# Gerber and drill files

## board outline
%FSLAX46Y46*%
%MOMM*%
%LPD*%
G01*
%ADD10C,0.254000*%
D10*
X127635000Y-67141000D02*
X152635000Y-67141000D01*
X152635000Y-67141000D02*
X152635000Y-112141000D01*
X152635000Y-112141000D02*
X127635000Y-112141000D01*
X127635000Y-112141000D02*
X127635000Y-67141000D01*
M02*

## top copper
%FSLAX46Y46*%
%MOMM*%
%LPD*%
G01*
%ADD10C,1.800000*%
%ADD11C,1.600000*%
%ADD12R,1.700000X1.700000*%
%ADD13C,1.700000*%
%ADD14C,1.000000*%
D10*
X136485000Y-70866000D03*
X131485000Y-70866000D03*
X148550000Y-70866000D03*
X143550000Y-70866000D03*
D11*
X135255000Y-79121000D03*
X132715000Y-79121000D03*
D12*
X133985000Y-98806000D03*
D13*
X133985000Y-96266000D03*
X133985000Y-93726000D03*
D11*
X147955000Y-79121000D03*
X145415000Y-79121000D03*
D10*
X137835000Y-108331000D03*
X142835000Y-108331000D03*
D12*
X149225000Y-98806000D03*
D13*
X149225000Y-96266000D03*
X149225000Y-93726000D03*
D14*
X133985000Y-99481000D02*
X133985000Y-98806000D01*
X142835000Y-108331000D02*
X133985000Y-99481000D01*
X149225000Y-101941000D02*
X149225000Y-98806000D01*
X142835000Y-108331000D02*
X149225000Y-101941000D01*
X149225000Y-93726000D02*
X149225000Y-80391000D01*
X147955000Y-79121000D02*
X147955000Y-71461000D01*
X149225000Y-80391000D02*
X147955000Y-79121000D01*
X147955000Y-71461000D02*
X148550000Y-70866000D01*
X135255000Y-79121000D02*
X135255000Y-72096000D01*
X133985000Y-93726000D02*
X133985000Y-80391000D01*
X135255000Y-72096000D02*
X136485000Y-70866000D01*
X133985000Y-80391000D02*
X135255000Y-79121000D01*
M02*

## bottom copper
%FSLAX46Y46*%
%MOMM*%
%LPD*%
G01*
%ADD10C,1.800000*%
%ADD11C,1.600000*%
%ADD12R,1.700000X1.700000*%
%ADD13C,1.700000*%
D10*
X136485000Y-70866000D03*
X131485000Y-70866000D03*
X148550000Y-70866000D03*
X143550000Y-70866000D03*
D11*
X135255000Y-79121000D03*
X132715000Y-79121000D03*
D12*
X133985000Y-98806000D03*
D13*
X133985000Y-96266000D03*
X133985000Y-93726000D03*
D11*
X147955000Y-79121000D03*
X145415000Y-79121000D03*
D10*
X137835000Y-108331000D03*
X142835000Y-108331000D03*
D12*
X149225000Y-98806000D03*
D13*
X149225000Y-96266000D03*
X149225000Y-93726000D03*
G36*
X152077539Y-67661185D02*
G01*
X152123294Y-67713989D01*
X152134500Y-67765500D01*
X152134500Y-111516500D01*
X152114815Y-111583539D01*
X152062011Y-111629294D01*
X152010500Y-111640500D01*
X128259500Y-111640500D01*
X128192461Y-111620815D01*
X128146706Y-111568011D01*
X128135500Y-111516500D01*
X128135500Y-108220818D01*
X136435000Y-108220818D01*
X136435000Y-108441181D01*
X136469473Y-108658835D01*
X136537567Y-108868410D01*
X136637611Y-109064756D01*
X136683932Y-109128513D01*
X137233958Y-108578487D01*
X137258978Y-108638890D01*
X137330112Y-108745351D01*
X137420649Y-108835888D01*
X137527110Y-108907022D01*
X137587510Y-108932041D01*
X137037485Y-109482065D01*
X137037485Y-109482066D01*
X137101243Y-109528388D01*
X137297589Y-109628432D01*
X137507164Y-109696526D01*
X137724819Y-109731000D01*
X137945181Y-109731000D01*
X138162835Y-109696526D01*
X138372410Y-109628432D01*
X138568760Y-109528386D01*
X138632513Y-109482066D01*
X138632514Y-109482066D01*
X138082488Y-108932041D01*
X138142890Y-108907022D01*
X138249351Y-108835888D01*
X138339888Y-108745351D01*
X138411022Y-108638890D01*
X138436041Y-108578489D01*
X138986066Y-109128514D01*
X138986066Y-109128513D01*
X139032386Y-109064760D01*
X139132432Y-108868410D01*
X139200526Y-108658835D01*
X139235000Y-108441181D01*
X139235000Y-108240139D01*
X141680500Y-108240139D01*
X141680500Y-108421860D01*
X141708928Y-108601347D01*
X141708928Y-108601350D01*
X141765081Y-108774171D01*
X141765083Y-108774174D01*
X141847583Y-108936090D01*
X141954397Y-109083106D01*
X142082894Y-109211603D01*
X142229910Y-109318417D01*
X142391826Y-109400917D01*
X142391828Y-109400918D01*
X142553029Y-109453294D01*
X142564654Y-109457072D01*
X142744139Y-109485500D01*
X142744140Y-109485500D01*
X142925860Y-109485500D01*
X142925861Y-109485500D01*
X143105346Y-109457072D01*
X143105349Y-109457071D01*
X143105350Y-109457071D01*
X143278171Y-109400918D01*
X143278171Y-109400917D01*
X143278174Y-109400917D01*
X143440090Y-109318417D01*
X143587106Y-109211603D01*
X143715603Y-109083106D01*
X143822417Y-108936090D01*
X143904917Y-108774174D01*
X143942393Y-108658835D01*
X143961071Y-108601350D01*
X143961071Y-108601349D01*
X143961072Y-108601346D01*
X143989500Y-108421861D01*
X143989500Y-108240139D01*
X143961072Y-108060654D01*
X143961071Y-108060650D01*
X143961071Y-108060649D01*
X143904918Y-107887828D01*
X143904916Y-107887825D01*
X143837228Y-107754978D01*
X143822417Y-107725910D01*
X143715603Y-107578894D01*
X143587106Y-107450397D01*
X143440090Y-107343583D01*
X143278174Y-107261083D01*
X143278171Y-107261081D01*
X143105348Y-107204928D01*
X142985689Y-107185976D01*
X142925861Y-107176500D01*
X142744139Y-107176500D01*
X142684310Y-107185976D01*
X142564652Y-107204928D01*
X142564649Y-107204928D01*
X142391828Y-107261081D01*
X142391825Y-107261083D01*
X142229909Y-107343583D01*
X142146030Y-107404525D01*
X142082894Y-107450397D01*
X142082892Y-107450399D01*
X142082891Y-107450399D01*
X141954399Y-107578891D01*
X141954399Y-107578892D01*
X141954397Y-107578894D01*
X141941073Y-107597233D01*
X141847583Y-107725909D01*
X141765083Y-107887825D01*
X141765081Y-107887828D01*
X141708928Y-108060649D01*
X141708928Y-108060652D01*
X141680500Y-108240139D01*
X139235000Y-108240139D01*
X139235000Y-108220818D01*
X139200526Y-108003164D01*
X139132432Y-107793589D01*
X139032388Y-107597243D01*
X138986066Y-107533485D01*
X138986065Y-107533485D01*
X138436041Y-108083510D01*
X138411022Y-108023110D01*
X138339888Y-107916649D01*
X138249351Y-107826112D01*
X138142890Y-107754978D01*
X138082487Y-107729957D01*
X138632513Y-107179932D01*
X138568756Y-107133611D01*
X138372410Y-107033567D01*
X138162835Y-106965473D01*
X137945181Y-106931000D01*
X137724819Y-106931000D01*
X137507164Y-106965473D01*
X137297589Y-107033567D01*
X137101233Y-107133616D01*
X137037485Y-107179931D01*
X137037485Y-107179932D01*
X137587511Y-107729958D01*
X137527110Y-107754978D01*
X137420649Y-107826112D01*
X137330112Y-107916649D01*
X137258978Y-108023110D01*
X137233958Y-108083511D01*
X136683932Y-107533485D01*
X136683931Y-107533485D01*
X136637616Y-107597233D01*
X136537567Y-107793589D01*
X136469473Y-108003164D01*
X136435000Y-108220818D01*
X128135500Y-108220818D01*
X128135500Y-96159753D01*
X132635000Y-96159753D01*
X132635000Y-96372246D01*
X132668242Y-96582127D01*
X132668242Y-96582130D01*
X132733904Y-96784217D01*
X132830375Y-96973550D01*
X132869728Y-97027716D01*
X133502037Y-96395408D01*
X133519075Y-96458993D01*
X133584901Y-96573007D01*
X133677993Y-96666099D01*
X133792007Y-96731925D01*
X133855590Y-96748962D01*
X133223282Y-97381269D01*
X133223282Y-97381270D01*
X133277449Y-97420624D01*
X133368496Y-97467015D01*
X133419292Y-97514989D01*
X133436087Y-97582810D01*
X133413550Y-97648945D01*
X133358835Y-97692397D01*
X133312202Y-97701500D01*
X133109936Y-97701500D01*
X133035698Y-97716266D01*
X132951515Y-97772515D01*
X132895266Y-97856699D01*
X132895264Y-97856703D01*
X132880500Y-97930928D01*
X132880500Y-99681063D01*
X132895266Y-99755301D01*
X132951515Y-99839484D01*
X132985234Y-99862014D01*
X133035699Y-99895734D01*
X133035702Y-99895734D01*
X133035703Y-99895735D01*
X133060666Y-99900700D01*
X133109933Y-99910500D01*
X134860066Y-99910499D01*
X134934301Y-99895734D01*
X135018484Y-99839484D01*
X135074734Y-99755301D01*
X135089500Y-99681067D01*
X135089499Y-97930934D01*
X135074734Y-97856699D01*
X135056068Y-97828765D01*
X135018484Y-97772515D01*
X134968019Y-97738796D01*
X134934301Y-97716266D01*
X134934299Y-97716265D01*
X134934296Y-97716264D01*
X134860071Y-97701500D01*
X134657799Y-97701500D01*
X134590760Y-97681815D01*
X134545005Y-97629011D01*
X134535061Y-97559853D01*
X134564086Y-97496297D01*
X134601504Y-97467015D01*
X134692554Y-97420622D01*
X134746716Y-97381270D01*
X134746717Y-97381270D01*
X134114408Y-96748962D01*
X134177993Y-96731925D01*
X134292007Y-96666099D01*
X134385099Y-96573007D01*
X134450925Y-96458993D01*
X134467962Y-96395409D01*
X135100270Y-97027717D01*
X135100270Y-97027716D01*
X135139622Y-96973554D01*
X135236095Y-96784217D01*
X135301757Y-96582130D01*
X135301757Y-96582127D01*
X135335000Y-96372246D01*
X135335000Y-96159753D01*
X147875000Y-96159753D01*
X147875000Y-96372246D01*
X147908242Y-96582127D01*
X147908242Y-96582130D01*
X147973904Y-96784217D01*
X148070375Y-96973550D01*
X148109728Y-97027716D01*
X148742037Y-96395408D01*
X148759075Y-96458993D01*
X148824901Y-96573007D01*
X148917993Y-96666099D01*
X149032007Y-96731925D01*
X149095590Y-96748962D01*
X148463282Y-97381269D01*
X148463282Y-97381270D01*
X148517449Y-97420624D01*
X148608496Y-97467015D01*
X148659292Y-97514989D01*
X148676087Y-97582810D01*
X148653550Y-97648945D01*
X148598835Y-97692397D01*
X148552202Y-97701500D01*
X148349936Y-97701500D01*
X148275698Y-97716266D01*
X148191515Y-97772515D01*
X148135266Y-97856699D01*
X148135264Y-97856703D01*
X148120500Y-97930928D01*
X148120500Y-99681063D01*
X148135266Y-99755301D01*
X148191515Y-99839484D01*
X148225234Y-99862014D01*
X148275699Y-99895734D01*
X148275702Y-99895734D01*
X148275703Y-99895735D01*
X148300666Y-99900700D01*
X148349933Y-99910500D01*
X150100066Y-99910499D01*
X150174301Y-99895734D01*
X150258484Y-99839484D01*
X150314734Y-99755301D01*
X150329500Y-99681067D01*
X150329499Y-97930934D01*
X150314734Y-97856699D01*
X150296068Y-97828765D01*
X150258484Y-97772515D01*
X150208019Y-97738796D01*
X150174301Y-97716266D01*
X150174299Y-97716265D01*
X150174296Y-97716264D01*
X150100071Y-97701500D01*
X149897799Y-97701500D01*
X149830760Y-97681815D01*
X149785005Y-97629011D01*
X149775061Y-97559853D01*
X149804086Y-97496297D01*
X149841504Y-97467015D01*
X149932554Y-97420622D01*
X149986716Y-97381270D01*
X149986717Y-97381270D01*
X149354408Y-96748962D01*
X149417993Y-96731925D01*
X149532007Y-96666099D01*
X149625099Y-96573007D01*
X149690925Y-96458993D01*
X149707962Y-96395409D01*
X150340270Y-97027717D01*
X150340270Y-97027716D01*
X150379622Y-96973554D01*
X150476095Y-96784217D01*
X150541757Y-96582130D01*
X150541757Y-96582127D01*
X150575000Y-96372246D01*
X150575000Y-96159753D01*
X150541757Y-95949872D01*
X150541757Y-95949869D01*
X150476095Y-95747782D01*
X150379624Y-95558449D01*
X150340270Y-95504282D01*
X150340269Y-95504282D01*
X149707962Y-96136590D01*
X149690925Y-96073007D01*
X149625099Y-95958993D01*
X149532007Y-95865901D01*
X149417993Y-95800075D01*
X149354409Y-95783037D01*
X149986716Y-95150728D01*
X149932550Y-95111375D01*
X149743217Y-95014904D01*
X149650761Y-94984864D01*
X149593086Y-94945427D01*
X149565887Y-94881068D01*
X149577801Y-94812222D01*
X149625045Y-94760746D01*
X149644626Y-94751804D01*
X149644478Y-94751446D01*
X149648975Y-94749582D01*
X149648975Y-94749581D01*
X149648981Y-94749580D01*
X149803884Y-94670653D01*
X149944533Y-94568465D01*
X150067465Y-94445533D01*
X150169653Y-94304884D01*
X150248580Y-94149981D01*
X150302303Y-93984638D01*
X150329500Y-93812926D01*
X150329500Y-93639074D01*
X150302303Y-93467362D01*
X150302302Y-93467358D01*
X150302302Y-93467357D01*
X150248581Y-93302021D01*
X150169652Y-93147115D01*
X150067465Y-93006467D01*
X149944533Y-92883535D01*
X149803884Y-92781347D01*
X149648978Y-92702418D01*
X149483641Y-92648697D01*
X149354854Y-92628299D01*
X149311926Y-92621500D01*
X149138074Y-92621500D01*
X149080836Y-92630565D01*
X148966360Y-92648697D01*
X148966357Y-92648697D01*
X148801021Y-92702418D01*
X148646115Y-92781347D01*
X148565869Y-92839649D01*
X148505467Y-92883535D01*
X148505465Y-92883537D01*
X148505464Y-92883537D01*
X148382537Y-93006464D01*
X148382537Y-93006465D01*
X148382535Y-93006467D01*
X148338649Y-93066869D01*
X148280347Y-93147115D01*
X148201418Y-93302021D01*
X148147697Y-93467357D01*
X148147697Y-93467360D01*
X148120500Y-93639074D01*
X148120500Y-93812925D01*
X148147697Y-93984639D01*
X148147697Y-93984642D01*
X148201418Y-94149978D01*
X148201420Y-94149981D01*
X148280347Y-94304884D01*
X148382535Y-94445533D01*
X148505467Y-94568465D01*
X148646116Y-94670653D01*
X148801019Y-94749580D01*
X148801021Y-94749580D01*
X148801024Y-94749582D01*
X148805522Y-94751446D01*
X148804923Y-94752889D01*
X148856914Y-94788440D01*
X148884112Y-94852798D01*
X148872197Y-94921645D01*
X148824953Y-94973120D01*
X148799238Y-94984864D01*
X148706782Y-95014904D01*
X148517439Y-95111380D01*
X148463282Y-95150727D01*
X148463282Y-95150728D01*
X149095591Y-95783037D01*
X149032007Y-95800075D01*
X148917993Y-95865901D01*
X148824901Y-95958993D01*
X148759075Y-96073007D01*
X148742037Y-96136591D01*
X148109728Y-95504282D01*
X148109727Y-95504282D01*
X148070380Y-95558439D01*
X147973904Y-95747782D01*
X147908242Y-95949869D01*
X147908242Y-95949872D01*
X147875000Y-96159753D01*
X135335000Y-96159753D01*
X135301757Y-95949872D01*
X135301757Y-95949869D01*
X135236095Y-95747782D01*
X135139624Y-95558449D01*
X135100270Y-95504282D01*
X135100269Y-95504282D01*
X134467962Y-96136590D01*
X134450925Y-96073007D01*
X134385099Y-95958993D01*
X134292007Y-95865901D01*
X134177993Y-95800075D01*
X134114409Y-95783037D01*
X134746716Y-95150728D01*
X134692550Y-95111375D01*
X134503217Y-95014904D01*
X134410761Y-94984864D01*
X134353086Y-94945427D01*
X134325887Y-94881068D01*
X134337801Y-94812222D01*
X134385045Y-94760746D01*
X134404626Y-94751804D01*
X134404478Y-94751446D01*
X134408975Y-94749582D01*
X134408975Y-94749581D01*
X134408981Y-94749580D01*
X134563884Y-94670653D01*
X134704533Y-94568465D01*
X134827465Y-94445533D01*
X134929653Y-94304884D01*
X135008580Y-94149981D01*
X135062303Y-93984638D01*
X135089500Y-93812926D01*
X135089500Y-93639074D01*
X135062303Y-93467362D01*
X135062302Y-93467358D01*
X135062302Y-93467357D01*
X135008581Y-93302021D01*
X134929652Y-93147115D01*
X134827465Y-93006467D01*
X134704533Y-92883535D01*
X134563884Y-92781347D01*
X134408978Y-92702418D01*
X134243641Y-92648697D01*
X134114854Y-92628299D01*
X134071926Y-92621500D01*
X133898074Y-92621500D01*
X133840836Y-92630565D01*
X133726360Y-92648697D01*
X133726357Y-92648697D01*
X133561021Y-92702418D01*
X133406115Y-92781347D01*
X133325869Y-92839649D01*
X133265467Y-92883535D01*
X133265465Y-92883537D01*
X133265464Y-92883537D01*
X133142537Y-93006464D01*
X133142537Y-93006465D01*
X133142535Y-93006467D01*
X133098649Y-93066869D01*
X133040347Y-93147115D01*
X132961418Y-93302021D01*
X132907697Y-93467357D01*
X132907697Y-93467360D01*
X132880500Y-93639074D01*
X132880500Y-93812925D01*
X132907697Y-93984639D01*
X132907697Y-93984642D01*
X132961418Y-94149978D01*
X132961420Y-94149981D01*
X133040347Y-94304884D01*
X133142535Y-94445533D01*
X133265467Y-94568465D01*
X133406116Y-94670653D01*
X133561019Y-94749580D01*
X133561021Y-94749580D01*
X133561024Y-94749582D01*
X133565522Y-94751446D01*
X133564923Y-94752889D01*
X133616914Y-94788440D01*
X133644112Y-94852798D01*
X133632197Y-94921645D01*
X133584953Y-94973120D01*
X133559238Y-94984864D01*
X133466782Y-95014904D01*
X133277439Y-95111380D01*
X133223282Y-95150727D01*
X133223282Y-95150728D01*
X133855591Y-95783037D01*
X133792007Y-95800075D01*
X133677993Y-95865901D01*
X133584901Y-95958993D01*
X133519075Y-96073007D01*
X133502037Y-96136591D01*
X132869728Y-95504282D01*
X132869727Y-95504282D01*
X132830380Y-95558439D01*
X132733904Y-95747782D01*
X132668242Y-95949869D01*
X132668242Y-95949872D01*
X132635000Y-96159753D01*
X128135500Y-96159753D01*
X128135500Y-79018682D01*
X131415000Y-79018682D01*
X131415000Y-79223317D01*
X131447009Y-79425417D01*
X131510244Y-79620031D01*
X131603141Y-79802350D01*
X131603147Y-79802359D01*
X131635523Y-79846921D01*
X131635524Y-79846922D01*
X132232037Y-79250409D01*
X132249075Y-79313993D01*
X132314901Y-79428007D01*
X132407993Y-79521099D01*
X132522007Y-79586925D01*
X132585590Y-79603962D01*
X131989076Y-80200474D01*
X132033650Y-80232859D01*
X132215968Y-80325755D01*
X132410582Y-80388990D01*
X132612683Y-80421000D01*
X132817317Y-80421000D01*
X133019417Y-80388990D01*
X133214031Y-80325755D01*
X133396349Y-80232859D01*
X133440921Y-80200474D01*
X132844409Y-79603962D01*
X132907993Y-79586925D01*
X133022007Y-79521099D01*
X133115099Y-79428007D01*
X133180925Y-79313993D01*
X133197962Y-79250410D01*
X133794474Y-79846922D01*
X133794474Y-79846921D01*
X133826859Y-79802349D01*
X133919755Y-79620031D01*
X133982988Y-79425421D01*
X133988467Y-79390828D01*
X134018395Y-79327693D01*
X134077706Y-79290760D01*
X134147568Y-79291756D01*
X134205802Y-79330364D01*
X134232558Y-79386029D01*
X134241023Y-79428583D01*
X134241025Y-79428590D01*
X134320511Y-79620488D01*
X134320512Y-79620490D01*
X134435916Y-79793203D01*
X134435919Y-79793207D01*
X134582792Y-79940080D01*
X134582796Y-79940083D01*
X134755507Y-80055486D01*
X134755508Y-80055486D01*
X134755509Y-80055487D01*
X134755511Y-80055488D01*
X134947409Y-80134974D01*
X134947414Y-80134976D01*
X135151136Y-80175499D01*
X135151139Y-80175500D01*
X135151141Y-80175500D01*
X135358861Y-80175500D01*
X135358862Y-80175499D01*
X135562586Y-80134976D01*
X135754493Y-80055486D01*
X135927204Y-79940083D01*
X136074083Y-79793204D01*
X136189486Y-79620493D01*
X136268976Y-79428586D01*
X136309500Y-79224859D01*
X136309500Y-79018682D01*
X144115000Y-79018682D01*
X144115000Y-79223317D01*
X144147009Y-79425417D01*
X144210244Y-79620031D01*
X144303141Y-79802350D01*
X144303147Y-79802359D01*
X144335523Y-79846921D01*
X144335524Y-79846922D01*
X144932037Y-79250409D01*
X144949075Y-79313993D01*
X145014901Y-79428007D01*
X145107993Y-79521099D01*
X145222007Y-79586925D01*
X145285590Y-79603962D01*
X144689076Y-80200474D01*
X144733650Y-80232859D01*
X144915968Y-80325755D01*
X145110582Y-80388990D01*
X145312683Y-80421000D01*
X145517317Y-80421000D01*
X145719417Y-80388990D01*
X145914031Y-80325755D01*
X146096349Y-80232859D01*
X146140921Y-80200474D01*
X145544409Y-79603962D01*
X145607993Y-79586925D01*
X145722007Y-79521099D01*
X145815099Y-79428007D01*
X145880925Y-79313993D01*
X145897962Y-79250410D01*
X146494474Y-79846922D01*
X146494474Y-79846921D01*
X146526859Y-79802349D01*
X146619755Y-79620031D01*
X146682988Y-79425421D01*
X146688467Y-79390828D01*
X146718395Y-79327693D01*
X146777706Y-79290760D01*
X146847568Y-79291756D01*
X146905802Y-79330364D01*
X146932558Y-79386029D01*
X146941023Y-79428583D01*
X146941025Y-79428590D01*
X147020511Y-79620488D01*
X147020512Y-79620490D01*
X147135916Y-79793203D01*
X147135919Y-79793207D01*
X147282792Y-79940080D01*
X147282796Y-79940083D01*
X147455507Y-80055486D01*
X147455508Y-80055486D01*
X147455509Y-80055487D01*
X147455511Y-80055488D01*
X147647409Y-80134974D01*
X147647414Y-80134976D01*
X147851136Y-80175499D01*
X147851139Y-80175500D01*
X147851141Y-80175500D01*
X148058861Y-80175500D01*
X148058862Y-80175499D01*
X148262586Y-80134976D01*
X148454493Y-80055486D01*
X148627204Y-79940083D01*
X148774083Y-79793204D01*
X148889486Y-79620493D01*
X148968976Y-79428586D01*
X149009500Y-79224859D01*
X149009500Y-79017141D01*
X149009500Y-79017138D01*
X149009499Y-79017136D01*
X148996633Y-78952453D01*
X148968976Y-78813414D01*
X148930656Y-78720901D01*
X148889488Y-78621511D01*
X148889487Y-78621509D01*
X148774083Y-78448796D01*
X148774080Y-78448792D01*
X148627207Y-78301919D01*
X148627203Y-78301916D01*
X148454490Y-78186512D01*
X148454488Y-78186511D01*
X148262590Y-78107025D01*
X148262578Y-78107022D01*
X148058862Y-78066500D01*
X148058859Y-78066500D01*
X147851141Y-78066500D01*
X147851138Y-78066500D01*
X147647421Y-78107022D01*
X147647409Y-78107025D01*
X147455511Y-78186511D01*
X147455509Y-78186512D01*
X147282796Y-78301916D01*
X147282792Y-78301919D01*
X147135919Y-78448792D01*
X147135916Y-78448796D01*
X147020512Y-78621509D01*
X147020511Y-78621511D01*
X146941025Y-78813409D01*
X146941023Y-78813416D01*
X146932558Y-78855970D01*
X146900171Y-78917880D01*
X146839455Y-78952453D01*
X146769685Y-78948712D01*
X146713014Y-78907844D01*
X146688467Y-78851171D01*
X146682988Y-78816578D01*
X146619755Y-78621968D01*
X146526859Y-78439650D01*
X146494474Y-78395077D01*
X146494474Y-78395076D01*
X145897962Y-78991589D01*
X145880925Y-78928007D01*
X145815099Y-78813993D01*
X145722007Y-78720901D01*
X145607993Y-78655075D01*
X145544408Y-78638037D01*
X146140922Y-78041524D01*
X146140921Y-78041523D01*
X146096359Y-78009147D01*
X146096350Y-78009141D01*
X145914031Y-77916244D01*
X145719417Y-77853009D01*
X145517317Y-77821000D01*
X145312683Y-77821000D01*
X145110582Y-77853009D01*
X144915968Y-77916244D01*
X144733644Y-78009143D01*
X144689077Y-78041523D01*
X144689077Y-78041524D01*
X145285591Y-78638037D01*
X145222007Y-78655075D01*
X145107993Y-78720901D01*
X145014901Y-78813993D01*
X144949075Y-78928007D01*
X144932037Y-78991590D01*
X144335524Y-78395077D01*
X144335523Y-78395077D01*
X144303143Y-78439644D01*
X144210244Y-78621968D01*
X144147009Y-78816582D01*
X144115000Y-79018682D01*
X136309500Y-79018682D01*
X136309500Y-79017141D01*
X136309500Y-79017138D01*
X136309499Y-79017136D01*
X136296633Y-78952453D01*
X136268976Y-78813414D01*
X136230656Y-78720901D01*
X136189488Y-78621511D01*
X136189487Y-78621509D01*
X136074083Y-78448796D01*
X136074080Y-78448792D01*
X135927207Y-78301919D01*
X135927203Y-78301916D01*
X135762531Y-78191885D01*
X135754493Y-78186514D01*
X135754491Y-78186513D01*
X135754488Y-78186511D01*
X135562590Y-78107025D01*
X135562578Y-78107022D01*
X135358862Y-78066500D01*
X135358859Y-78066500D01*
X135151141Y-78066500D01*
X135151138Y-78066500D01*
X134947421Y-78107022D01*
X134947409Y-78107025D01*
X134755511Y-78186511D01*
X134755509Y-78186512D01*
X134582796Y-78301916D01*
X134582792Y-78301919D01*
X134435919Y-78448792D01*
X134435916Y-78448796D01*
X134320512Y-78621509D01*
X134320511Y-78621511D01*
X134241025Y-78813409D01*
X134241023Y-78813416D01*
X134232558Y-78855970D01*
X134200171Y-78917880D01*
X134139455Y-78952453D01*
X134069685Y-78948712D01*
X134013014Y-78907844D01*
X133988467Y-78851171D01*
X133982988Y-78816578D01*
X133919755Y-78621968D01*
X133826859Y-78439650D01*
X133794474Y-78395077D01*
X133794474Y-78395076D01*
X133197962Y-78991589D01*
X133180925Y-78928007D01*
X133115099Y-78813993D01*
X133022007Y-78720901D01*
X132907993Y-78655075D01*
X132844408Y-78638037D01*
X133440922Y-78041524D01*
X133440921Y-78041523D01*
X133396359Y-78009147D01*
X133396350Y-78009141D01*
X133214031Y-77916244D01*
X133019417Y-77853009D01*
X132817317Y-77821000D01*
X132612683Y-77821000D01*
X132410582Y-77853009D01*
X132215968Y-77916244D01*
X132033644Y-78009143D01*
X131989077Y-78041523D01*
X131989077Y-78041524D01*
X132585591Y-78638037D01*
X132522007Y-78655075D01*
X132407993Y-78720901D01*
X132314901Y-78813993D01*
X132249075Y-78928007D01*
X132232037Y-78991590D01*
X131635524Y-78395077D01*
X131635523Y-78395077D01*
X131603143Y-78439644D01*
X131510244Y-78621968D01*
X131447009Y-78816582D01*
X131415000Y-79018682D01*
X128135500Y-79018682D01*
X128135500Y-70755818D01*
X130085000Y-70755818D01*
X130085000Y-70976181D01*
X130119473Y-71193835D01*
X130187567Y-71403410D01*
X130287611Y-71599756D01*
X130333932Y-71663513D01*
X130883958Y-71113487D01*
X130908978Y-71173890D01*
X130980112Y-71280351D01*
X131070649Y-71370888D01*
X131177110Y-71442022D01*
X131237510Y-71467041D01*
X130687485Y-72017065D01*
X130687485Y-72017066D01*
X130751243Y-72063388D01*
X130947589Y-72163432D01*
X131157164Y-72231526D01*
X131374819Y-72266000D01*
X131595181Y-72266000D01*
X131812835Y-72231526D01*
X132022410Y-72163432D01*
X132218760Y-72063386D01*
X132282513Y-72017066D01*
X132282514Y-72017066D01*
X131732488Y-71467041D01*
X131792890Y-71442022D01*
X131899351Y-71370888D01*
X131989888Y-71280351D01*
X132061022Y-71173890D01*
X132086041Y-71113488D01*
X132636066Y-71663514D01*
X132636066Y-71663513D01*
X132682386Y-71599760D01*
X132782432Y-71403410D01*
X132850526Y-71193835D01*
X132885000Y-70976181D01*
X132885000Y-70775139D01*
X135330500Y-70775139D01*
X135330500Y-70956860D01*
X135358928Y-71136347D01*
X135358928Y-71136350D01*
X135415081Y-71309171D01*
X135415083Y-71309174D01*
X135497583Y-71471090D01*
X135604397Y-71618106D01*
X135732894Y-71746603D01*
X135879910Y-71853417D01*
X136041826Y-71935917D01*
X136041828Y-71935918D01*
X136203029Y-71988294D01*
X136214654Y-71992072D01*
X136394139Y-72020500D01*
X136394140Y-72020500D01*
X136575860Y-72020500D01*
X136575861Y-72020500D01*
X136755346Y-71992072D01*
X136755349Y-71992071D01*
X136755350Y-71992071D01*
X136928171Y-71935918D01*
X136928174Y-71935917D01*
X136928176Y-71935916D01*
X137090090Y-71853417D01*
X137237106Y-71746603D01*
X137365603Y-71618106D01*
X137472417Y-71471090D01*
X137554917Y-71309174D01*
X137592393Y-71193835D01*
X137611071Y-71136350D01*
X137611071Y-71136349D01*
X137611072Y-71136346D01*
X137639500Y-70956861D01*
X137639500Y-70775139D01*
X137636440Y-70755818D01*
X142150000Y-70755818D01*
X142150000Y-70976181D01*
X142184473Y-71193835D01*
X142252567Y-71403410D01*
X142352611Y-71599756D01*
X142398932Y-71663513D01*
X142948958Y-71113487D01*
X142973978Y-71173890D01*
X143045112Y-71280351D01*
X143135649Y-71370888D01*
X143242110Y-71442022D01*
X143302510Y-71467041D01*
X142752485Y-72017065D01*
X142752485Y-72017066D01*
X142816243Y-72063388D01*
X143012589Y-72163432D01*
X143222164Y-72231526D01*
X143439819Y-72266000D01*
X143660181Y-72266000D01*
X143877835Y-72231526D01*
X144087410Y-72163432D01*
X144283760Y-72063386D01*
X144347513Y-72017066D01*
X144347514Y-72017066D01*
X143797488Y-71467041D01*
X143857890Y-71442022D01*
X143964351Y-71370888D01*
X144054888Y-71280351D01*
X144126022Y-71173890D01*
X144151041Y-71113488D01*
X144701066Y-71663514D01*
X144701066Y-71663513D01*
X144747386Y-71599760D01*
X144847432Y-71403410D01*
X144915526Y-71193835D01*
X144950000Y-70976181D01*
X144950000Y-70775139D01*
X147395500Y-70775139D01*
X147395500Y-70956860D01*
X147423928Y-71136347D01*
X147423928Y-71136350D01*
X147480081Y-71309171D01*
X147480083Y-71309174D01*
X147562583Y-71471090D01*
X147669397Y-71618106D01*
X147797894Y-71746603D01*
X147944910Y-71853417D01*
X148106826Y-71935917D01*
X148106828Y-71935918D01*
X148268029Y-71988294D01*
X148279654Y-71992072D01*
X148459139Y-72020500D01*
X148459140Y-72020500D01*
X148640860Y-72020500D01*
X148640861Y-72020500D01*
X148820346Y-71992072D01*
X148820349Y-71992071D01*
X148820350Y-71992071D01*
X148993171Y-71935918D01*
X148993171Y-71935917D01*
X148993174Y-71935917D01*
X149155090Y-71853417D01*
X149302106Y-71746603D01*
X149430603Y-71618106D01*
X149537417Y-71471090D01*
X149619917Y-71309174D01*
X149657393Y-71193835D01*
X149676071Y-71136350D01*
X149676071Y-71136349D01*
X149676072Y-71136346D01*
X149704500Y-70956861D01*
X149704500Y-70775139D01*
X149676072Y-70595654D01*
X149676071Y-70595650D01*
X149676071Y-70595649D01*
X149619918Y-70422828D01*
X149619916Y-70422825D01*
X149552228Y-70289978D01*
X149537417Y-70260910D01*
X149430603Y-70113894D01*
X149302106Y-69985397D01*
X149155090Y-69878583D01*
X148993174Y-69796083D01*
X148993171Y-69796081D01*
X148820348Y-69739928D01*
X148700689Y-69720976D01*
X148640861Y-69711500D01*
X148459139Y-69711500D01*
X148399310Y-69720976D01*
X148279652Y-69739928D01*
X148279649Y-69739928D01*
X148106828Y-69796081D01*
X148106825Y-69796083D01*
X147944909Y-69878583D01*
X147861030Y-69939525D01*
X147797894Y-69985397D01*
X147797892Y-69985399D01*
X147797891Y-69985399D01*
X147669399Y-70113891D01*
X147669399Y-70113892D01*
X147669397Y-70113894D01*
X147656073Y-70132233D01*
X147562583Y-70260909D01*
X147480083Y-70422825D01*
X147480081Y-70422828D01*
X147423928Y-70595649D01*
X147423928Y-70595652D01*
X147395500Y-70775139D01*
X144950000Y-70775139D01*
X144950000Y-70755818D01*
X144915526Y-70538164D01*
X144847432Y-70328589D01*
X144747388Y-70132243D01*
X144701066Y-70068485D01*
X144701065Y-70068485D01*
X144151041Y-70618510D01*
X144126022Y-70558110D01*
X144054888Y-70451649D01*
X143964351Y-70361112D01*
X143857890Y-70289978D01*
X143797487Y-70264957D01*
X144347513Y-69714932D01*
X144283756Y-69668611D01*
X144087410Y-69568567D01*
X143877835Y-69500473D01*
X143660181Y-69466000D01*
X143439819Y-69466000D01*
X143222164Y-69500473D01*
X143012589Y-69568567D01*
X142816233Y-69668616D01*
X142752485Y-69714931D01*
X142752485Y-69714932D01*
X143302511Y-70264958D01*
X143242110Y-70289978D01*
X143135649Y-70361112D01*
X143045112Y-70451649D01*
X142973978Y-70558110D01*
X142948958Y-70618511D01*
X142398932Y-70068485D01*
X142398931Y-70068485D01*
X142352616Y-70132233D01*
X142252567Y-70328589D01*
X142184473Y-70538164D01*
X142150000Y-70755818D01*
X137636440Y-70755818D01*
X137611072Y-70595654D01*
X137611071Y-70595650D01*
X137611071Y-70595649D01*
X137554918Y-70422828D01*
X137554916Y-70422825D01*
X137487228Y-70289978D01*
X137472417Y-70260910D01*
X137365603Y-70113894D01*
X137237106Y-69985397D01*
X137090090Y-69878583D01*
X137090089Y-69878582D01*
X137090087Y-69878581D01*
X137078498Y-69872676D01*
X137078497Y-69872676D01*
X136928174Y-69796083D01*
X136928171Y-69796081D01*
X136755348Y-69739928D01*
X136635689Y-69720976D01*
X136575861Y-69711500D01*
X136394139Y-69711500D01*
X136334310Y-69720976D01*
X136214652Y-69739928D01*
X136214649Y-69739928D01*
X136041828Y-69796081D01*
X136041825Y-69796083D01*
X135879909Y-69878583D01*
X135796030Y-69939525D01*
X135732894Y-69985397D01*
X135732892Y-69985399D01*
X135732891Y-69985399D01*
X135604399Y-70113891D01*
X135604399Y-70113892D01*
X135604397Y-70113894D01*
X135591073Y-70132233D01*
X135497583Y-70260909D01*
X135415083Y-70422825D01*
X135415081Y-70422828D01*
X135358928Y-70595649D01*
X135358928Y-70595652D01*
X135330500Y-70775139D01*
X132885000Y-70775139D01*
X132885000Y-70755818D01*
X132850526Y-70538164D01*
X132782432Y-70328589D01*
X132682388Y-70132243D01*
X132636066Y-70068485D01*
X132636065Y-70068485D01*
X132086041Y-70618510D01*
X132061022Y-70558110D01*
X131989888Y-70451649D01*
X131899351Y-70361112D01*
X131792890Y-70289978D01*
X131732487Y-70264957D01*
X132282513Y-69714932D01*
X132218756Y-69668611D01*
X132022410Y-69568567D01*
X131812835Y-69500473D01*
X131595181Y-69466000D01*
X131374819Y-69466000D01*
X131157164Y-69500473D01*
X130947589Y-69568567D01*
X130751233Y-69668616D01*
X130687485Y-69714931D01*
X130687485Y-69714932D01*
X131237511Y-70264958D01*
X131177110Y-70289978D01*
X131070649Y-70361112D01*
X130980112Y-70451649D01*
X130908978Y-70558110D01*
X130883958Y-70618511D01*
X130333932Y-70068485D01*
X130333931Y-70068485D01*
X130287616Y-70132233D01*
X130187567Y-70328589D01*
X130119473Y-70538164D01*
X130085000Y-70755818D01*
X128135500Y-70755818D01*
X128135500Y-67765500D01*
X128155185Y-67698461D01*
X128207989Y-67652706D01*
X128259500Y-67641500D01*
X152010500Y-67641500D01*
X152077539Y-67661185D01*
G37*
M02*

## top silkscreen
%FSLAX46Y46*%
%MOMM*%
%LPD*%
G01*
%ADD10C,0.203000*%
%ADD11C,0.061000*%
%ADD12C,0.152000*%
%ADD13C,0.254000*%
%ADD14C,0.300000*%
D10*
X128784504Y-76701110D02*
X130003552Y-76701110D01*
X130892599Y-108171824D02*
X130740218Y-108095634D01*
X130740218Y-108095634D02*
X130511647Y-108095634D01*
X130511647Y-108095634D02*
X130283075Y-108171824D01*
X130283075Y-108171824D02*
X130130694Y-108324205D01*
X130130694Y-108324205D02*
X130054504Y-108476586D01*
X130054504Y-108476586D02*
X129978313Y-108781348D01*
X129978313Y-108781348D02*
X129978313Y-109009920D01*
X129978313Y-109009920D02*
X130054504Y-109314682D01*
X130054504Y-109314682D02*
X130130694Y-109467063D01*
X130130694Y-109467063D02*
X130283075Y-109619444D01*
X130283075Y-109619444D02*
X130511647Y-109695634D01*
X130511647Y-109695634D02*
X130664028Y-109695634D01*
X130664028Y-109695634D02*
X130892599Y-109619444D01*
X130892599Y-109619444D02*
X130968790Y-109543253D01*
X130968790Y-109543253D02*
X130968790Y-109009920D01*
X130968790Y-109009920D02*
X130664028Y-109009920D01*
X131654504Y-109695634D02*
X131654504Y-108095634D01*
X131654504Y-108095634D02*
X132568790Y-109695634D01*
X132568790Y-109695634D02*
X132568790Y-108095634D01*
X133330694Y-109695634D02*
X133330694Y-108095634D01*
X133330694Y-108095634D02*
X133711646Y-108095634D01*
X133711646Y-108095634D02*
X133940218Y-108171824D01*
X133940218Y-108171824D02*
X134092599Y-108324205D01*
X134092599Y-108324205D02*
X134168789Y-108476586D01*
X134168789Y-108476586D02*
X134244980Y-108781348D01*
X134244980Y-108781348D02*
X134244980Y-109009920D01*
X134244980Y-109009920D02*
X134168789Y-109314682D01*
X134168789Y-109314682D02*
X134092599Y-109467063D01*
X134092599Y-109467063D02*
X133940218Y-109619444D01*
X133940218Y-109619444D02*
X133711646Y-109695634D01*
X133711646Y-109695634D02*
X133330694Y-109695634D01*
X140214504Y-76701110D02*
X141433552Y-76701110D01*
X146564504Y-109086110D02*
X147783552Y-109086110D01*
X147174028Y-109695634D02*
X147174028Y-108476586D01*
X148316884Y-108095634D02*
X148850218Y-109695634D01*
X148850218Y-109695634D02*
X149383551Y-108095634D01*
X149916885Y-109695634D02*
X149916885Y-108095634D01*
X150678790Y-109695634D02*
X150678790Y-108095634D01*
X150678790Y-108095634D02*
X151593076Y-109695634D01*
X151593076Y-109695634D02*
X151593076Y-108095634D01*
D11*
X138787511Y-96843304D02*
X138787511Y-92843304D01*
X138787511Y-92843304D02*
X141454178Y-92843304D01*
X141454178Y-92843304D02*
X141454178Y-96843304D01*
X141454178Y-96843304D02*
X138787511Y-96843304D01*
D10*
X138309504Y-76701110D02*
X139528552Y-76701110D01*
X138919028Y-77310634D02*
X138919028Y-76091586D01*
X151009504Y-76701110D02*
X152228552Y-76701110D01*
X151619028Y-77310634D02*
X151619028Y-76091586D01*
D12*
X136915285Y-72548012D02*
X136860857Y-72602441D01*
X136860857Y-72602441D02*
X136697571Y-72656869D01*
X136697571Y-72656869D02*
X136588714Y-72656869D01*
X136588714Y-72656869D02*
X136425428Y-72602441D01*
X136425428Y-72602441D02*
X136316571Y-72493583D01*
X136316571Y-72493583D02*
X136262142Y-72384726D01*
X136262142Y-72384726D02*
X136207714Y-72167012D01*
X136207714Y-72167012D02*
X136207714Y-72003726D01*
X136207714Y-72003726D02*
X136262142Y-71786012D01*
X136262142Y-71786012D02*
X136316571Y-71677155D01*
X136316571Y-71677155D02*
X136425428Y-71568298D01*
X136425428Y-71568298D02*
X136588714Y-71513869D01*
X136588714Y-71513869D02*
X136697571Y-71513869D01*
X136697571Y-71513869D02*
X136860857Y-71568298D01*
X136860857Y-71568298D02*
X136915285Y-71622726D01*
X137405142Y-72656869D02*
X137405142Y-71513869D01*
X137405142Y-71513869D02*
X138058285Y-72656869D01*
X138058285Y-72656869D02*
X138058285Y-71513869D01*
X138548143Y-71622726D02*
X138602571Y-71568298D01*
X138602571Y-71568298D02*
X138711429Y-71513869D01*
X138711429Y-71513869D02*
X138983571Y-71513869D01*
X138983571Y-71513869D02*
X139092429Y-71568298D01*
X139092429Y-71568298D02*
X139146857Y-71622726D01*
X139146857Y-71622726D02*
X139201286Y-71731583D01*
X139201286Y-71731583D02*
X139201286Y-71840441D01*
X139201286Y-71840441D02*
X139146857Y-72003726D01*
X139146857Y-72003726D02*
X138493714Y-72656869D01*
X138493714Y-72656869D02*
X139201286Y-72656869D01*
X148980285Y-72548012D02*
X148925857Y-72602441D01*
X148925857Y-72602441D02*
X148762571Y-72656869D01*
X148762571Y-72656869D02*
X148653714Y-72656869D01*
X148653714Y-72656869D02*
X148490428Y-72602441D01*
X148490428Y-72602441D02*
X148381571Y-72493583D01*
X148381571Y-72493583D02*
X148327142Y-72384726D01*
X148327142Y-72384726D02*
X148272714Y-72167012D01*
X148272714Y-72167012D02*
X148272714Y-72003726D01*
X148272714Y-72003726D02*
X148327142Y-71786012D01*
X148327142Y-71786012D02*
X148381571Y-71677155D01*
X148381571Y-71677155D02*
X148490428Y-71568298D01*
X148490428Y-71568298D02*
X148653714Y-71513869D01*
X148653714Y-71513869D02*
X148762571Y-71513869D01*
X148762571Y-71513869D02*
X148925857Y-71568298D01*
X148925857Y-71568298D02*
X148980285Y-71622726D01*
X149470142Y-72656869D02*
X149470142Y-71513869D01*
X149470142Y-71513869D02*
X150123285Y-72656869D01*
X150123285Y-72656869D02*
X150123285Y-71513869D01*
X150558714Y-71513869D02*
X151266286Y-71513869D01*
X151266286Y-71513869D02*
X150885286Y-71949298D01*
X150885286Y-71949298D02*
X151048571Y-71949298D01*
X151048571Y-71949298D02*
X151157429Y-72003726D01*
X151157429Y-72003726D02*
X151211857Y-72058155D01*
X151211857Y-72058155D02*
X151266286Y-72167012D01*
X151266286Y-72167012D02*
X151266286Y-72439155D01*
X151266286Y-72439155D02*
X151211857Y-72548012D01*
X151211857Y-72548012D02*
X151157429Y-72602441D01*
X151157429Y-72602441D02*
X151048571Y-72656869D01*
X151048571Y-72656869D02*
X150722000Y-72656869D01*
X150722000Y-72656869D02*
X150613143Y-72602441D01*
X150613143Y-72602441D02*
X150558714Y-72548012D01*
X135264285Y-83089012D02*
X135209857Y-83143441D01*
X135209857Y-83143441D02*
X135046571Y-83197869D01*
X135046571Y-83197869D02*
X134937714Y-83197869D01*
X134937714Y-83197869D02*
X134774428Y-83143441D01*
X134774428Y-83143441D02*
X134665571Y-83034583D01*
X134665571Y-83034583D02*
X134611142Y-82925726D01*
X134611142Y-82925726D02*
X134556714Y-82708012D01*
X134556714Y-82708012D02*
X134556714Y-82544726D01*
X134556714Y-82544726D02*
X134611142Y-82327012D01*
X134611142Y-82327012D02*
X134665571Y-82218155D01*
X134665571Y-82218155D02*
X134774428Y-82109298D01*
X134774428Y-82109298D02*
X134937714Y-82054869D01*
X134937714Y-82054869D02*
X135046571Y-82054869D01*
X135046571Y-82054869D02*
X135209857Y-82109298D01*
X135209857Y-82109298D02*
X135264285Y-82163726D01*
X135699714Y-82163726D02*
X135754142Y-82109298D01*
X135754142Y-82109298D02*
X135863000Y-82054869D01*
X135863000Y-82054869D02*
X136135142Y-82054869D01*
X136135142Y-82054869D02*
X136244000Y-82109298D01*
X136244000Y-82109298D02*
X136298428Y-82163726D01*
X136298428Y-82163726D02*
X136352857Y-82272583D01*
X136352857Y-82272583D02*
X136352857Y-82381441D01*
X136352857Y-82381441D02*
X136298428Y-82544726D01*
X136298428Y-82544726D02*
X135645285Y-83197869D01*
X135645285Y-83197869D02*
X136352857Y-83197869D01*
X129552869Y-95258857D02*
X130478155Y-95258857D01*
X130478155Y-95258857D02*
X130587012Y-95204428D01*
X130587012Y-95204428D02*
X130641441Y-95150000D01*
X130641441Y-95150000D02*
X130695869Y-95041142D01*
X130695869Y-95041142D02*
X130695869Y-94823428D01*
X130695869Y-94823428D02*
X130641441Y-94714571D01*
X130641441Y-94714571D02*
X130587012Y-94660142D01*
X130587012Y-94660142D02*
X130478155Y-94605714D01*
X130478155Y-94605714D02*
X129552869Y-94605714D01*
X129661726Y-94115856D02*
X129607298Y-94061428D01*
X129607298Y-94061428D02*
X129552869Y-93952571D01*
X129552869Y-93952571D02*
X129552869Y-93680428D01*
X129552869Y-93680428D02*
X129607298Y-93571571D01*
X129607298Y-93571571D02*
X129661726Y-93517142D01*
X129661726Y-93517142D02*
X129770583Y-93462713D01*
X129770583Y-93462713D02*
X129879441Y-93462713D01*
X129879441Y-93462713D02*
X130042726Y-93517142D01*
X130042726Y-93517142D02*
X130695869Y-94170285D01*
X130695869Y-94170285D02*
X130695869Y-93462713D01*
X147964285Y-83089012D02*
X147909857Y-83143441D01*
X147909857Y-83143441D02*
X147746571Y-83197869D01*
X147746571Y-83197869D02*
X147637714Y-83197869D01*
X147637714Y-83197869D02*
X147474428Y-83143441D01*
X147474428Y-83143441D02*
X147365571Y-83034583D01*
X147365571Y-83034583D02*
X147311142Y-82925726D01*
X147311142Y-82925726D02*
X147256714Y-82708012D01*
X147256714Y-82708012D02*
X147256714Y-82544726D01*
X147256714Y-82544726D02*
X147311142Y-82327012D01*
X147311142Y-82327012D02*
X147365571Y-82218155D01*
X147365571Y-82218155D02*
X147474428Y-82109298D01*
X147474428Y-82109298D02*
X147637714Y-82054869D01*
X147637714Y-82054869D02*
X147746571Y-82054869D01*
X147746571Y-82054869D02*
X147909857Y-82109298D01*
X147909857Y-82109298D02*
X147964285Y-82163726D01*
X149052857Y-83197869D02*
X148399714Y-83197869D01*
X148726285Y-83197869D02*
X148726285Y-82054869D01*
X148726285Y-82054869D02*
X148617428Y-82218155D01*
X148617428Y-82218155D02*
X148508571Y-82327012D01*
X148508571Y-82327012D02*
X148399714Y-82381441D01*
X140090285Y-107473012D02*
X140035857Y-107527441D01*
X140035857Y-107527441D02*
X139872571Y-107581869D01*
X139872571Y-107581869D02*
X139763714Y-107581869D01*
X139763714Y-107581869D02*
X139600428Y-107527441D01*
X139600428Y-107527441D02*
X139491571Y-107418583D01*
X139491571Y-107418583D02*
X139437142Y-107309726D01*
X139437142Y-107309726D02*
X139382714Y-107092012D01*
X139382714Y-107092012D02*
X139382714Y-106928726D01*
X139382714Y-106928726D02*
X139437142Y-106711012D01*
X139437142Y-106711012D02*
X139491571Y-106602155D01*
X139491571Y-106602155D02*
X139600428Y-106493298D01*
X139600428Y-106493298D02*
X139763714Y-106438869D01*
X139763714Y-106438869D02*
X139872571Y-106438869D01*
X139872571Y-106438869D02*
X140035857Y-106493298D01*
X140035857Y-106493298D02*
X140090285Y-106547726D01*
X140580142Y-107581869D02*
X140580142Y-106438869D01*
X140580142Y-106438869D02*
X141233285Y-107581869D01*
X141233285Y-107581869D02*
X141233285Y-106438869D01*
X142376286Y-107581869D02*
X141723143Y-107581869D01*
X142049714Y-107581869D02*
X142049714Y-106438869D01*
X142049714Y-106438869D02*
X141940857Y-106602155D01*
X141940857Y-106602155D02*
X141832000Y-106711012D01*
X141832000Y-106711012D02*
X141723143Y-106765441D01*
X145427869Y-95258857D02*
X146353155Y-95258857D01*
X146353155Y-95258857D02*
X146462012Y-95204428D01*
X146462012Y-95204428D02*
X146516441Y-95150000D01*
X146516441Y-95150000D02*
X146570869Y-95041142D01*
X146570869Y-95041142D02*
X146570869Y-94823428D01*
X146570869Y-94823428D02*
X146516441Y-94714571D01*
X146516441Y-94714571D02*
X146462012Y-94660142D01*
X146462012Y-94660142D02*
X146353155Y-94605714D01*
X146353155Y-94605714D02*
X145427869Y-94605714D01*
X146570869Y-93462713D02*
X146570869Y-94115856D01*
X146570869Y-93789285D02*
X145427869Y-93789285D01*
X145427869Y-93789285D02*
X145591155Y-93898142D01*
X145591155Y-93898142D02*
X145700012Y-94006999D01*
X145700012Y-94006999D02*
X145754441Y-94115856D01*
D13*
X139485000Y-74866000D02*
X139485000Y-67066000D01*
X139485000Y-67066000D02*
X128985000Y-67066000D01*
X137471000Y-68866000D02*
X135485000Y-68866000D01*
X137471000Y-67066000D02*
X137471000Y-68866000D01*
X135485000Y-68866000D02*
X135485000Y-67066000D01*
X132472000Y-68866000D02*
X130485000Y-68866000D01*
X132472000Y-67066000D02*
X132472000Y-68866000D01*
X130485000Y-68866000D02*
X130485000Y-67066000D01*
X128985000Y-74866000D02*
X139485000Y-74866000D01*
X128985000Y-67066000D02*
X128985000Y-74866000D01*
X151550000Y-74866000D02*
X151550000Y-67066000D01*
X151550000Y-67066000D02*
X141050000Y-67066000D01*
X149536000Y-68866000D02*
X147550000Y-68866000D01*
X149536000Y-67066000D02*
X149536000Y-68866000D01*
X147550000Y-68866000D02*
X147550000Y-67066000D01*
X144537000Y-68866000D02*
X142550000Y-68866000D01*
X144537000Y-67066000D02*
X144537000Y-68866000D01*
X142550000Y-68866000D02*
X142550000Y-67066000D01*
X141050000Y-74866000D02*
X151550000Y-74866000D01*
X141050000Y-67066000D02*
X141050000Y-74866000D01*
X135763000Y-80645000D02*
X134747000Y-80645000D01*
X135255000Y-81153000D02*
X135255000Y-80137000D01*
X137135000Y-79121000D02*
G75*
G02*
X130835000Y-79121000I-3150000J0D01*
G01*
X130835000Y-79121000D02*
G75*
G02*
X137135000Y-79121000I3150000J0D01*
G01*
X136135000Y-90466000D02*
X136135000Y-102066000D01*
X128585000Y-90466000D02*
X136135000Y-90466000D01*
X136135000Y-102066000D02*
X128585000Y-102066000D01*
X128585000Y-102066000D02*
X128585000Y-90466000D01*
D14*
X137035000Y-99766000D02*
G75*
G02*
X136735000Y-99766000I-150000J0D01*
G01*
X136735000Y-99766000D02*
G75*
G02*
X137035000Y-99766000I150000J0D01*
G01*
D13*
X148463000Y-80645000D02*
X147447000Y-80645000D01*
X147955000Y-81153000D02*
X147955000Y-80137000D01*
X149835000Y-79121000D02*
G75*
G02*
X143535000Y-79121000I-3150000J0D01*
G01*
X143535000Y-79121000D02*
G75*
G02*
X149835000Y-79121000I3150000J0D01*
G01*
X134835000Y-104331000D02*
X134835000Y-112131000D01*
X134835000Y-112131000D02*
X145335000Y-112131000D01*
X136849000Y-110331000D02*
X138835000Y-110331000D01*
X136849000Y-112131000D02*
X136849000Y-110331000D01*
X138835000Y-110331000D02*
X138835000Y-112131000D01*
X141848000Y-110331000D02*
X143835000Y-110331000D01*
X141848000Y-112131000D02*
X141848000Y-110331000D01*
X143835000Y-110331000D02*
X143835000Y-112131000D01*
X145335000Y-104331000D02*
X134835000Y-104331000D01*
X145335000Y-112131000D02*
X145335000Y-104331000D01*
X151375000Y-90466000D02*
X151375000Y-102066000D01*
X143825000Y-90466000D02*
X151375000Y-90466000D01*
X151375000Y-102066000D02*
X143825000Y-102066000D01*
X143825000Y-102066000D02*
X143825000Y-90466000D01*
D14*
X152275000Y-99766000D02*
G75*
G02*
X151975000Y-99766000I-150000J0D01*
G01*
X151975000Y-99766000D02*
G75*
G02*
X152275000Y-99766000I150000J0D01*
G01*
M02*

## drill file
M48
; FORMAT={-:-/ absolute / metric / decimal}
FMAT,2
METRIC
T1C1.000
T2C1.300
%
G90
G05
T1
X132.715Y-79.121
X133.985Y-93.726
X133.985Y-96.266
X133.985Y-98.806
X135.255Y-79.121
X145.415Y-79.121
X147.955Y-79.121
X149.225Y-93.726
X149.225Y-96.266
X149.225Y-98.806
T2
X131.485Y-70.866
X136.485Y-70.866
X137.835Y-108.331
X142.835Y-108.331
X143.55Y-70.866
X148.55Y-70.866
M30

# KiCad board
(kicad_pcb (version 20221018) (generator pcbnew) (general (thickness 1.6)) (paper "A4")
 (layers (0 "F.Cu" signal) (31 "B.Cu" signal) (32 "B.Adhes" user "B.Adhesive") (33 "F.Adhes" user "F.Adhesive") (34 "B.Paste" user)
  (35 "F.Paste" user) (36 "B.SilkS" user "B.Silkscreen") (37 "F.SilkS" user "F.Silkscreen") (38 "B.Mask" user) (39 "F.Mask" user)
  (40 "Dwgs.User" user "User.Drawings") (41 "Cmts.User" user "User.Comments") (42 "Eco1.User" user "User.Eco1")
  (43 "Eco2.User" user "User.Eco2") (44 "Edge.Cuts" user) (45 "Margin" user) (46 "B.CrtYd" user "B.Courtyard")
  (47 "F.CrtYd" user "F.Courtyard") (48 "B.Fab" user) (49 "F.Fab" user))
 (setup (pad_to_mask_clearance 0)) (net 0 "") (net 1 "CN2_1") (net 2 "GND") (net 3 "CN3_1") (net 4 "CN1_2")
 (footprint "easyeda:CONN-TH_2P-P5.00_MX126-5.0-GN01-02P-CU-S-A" (layer "F.Cu") (at 133.985 70.866 180)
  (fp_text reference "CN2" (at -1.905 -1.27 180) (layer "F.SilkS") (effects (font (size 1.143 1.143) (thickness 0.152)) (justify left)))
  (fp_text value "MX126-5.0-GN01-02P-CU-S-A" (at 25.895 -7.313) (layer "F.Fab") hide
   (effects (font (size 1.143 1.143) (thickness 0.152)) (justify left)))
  (fp_line (start -5.5 -4) (end -5.5 3.8) (stroke (width 0.254) (type solid)) (layer "F.SilkS"))
  (fp_line (start -5.5 3.8) (end 5 3.8) (stroke (width 0.254) (type solid)) (layer "F.SilkS"))
  (fp_line (start -3.486 2) (end -1.5 2) (stroke (width 0.254) (type solid)) (layer "F.SilkS"))
  (fp_line (start -3.486 3.8) (end -3.486 2) (stroke (width 0.254) (type solid)) (layer "F.SilkS"))
  (fp_line (start -1.5 2) (end -1.5 3.8) (stroke (width 0.254) (type solid)) (layer "F.SilkS"))
  (fp_line (start 1.513 2) (end 3.5 2) (stroke (width 0.254) (type solid)) (layer "F.SilkS"))
  (fp_line (start 1.513 3.8) (end 1.513 2) (stroke (width 0.254) (type solid)) (layer "F.SilkS"))
  (fp_line (start 3.5 2) (end 3.5 3.8) (stroke (width 0.254) (type solid)) (layer "F.SilkS"))
  (fp_line (start 5 -4) (end -5.5 -4) (stroke (width 0.254) (type solid)) (layer "F.SilkS"))
  (fp_line (start 5 3.8) (end 5 -4) (stroke (width 0.254) (type solid)) (layer "F.SilkS"))
  (pad "1" thru_hole circle (at -2.5 0 180) (size 1.8 1.8) (drill 1.3) (layers "*.Cu" "*.Paste" "*.Mask") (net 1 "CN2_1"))
  (pad "2" thru_hole circle (at 2.5 0 180) (size 1.8 1.8) (drill 1.3) (layers "*.Cu" "*.Paste" "*.Mask") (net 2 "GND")))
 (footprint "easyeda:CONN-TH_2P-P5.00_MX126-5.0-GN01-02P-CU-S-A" (layer "F.Cu") (at 146.05 70.866 180)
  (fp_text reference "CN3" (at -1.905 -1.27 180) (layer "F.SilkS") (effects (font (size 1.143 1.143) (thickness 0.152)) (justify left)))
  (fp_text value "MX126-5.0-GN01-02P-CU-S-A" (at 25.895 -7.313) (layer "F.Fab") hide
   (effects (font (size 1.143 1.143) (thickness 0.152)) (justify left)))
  (fp_line (start -5.5 -4) (end -5.5 3.8) (stroke (width 0.254) (type solid)) (layer "F.SilkS"))
  (fp_line (start -5.5 3.8) (end 5 3.8) (stroke (width 0.254) (type solid)) (layer "F.SilkS"))
  (fp_line (start -3.486 2) (end -1.5 2) (stroke (width 0.254) (type solid)) (layer "F.SilkS"))
  (fp_line (start -3.486 3.8) (end -3.486 2) (stroke (width 0.254) (type solid)) (layer "F.SilkS"))
  (fp_line (start -1.5 2) (end -1.5 3.8) (stroke (width 0.254) (type solid)) (layer "F.SilkS"))
  (fp_line (start 1.513 2) (end 3.5 2) (stroke (width 0.254) (type solid)) (layer "F.SilkS"))
  (fp_line (start 1.513 3.8) (end 1.513 2) (stroke (width 0.254) (type solid)) (layer "F.SilkS"))
  (fp_line (start 3.5 2) (end 3.5 3.8) (stroke (width 0.254) (type solid)) (layer "F.SilkS"))
  (fp_line (start 5 -4) (end -5.5 -4) (stroke (width 0.254) (type solid)) (layer "F.SilkS"))
  (fp_line (start 5 3.8) (end 5 -4) (stroke (width 0.254) (type solid)) (layer "F.SilkS"))
  (pad "1" thru_hole circle (at -2.5 0 180) (size 1.8 1.8) (drill 1.3) (layers "*.Cu" "*.Paste" "*.Mask") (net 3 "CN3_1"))
  (pad "2" thru_hole circle (at 2.5 0 180) (size 1.8 1.8) (drill 1.3) (layers "*.Cu" "*.Paste" "*.Mask") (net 2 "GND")))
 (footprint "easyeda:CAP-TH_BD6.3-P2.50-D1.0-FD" (layer "F.Cu") (at 133.985 79.121 180)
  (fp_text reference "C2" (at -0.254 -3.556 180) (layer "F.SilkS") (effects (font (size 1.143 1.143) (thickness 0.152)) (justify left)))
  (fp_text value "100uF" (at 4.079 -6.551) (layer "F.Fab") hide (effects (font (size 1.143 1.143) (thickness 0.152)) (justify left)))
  (fp_line (start -1.778 -1.524) (end -0.762 -1.524) (stroke (width 0.254) (type solid)) (layer "F.SilkS"))
  (fp_line (start -1.27 -2.032) (end -1.27 -1.016) (stroke (width 0.254) (type solid)) (layer "F.SilkS"))
  (fp_circle (center 0 0) (end 3.15 0) (stroke (width 0.254) (type solid)) (fill none) (layer "F.SilkS"))
  (pad "1" thru_hole circle (at -1.27 0 180) (size 1.6 1.6) (drill 1) (layers "*.Cu" "*.Paste" "*.Mask") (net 1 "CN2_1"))
  (pad "2" thru_hole circle (at 1.27 0 180) (size 1.6 1.6) (drill 1) (layers "*.Cu" "*.Paste" "*.Mask") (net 2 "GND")))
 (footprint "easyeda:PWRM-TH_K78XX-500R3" (layer "F.Cu") (at 133.985 96.266 -90)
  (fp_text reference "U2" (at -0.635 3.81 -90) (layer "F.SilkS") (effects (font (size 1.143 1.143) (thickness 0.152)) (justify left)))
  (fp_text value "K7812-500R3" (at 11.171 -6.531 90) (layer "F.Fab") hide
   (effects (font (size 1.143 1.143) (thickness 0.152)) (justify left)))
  (fp_line (start -5.8 -2.15) (end 5.8 -2.15) (stroke (width 0.254) (type solid)) (layer "F.SilkS"))
  (fp_line (start -5.8 5.4) (end -5.8 -2.15) (stroke (width 0.254) (type solid)) (layer "F.SilkS"))
  (fp_line (start 5.8 -2.15) (end 5.8 5.4) (stroke (width 0.254) (type solid)) (layer "F.SilkS"))
  (fp_line (start 5.8 5.4) (end -5.8 5.4) (stroke (width 0.254) (type solid)) (layer "F.SilkS"))
  (fp_circle (center 3.5 -2.9) (end 3.65 -2.9) (stroke (width 0.3) (type solid)) (fill none) (layer "F.SilkS"))
  (pad "1" thru_hole rect (at 2.54 0 90) (size 1.7 1.7) (drill 1) (layers "*.Cu" "*.Paste" "*.Mask") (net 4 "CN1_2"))
  (pad "2" thru_hole circle (at 0 0 90) (size 1.7 1.7) (drill 1) (layers "*.Cu" "*.Paste" "*.Mask") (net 2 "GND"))
  (pad "3" thru_hole circle (at -2.54 0 90) (size 1.7 1.7) (drill 1) (layers "*.Cu" "*.Paste" "*.Mask") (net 1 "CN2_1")))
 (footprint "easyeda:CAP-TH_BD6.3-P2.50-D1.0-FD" (layer "F.Cu") (at 146.685 79.121 180)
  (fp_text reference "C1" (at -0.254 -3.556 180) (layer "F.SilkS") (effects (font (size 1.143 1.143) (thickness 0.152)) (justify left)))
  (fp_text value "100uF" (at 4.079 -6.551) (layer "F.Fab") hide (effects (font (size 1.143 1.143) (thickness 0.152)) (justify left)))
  (fp_line (start -1.778 -1.524) (end -0.762 -1.524) (stroke (width 0.254) (type solid)) (layer "F.SilkS"))
  (fp_line (start -1.27 -2.032) (end -1.27 -1.016) (stroke (width 0.254) (type solid)) (layer "F.SilkS"))
  (fp_circle (center 0 0) (end 3.15 0) (stroke (width 0.254) (type solid)) (fill none) (layer "F.SilkS"))
  (pad "1" thru_hole circle (at -1.27 0 180) (size 1.6 1.6) (drill 1) (layers "*.Cu" "*.Paste" "*.Mask") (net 3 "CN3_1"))
  (pad "2" thru_hole circle (at 1.27 0 180) (size 1.6 1.6) (drill 1) (layers "*.Cu" "*.Paste" "*.Mask") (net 2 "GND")))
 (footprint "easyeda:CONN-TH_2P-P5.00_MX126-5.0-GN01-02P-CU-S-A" (layer "F.Cu") (at 140.335 108.331)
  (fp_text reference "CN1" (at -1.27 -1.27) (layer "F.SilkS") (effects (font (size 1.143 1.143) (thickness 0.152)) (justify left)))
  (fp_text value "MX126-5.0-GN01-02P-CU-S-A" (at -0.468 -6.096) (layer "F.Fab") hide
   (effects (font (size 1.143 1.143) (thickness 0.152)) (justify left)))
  (fp_line (start -5.5 -4) (end -5.5 3.8) (stroke (width 0.254) (type solid)) (layer "F.SilkS"))
  (fp_line (start -5.5 3.8) (end 5 3.8) (stroke (width 0.254) (type solid)) (layer "F.SilkS"))
  (fp_line (start -3.486 2) (end -1.5 2) (stroke (width 0.254) (type solid)) (layer "F.SilkS"))
  (fp_line (start -3.486 3.8) (end -3.486 2) (stroke (width 0.254) (type solid)) (layer "F.SilkS"))
  (fp_line (start -1.5 2) (end -1.5 3.8) (stroke (width 0.254) (type solid)) (layer "F.SilkS"))
  (fp_line (start 1.513 2) (end 3.5 2) (stroke (width 0.254) (type solid)) (layer "F.SilkS"))
  (fp_line (start 1.513 3.8) (end 1.513 2) (stroke (width 0.254) (type solid)) (layer "F.SilkS"))
  (fp_line (start 3.5 2) (end 3.5 3.8) (stroke (width 0.254) (type solid)) (layer "F.SilkS"))
  (fp_line (start 5 -4) (end -5.5 -4) (stroke (width 0.254) (type solid)) (layer "F.SilkS"))
  (fp_line (start 5 3.8) (end 5 -4) (stroke (width 0.254) (type solid)) (layer "F.SilkS"))
  (pad "1" thru_hole circle (at -2.5 0) (size 1.8 1.8) (drill 1.3) (layers "*.Cu" "*.Paste" "*.Mask") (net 2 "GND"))
  (pad "2" thru_hole circle (at 2.5 0) (size 1.8 1.8) (drill 1.3) (layers "*.Cu" "*.Paste" "*.Mask") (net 4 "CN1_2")))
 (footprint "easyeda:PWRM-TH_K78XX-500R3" (layer "F.Cu") (at 149.225 96.266 -90)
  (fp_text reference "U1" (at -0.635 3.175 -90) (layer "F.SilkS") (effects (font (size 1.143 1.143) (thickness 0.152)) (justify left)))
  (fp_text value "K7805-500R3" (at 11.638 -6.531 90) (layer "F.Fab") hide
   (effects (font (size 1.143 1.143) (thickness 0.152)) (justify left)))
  (fp_line (start -5.8 -2.15) (end 5.8 -2.15) (stroke (width 0.254) (type solid)) (layer "F.SilkS"))
  (fp_line (start -5.8 5.4) (end -5.8 -2.15) (stroke (width 0.254) (type solid)) (layer "F.SilkS"))
  (fp_line (start 5.8 -2.15) (end 5.8 5.4) (stroke (width 0.254) (type solid)) (layer "F.SilkS"))
  (fp_line (start 5.8 5.4) (end -5.8 5.4) (stroke (width 0.254) (type solid)) (layer "F.SilkS"))
  (fp_circle (center 3.5 -2.9) (end 3.65 -2.9) (stroke (width 0.3) (type solid)) (fill none) (layer "F.SilkS"))
  (pad "1" thru_hole rect (at 2.54 0 90) (size 1.7 1.7) (drill 1) (layers "*.Cu" "*.Paste" "*.Mask") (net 4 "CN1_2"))
  (pad "2" thru_hole circle (at 0 0 90) (size 1.7 1.7) (drill 1) (layers "*.Cu" "*.Paste" "*.Mask") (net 2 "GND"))
  (pad "3" thru_hole circle (at -2.54 0 90) (size 1.7 1.7) (drill 1) (layers "*.Cu" "*.Paste" "*.Mask") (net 3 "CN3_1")))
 (gr_line (start 127.635 67.141) (end 152.635 67.141) (stroke (width 0.254) (type solid)) (layer "Edge.Cuts"))
 (gr_line (start 152.635 67.141) (end 152.635 112.141) (stroke (width 0.254) (type solid)) (layer "Edge.Cuts"))
 (gr_line (start 152.635 112.141) (end 127.635 112.141) (stroke (width 0.254) (type solid)) (layer "Edge.Cuts"))
 (gr_line (start 127.635 112.141) (end 127.635 67.141) (stroke (width 0.254) (type solid)) (layer "Edge.Cuts"))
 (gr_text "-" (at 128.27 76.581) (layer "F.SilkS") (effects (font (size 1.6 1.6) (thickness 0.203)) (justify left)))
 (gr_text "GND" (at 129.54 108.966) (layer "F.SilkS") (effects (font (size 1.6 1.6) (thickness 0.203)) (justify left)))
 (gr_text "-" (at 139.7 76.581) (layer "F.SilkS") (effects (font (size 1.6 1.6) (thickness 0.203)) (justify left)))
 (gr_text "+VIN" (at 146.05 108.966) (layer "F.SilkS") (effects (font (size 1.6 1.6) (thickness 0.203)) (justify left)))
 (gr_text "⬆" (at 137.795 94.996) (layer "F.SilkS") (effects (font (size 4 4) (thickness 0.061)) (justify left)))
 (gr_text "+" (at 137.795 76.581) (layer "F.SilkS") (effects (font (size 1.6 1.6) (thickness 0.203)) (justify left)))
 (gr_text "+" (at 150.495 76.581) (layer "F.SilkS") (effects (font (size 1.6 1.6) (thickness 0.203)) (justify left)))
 (segment (start 133.985 99.481) (end 133.985 98.806) (width 1) (layer "F.Cu") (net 4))
 (segment (start 142.835 108.331) (end 133.985 99.481) (width 1) (layer "F.Cu") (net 4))
 (segment (start 149.225 101.941) (end 149.225 98.806) (width 1) (layer "F.Cu") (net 4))
 (segment (start 142.835 108.331) (end 149.225 101.941) (width 1) (layer "F.Cu") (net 4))
 (segment (start 149.225 93.726) (end 149.225 80.391) (width 1) (layer "F.Cu") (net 3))
 (segment (start 147.955 79.121) (end 147.955 71.461) (width 1) (layer "F.Cu") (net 3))
 (segment (start 149.225 80.391) (end 147.955 79.121) (width 1) (layer "F.Cu") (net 3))
 (segment (start 147.955 71.461) (end 148.55 70.866) (width 1) (layer "F.Cu") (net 3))
 (segment (start 135.255 79.121) (end 135.255 72.096) (width 1) (layer "F.Cu") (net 1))
 (segment (start 133.985 93.726) (end 133.985 80.391) (width 1) (layer "F.Cu") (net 1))
 (segment (start 135.255 72.096) (end 136.485 70.866) (width 1) (layer "F.Cu") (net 1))
 (segment (start 133.985 80.391) (end 135.255 79.121) (width 1) (layer "F.Cu") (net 1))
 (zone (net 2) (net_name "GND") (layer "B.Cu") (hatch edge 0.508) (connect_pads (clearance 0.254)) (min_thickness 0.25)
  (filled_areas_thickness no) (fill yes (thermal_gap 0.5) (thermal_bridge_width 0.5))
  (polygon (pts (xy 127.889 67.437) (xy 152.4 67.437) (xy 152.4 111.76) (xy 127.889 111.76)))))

